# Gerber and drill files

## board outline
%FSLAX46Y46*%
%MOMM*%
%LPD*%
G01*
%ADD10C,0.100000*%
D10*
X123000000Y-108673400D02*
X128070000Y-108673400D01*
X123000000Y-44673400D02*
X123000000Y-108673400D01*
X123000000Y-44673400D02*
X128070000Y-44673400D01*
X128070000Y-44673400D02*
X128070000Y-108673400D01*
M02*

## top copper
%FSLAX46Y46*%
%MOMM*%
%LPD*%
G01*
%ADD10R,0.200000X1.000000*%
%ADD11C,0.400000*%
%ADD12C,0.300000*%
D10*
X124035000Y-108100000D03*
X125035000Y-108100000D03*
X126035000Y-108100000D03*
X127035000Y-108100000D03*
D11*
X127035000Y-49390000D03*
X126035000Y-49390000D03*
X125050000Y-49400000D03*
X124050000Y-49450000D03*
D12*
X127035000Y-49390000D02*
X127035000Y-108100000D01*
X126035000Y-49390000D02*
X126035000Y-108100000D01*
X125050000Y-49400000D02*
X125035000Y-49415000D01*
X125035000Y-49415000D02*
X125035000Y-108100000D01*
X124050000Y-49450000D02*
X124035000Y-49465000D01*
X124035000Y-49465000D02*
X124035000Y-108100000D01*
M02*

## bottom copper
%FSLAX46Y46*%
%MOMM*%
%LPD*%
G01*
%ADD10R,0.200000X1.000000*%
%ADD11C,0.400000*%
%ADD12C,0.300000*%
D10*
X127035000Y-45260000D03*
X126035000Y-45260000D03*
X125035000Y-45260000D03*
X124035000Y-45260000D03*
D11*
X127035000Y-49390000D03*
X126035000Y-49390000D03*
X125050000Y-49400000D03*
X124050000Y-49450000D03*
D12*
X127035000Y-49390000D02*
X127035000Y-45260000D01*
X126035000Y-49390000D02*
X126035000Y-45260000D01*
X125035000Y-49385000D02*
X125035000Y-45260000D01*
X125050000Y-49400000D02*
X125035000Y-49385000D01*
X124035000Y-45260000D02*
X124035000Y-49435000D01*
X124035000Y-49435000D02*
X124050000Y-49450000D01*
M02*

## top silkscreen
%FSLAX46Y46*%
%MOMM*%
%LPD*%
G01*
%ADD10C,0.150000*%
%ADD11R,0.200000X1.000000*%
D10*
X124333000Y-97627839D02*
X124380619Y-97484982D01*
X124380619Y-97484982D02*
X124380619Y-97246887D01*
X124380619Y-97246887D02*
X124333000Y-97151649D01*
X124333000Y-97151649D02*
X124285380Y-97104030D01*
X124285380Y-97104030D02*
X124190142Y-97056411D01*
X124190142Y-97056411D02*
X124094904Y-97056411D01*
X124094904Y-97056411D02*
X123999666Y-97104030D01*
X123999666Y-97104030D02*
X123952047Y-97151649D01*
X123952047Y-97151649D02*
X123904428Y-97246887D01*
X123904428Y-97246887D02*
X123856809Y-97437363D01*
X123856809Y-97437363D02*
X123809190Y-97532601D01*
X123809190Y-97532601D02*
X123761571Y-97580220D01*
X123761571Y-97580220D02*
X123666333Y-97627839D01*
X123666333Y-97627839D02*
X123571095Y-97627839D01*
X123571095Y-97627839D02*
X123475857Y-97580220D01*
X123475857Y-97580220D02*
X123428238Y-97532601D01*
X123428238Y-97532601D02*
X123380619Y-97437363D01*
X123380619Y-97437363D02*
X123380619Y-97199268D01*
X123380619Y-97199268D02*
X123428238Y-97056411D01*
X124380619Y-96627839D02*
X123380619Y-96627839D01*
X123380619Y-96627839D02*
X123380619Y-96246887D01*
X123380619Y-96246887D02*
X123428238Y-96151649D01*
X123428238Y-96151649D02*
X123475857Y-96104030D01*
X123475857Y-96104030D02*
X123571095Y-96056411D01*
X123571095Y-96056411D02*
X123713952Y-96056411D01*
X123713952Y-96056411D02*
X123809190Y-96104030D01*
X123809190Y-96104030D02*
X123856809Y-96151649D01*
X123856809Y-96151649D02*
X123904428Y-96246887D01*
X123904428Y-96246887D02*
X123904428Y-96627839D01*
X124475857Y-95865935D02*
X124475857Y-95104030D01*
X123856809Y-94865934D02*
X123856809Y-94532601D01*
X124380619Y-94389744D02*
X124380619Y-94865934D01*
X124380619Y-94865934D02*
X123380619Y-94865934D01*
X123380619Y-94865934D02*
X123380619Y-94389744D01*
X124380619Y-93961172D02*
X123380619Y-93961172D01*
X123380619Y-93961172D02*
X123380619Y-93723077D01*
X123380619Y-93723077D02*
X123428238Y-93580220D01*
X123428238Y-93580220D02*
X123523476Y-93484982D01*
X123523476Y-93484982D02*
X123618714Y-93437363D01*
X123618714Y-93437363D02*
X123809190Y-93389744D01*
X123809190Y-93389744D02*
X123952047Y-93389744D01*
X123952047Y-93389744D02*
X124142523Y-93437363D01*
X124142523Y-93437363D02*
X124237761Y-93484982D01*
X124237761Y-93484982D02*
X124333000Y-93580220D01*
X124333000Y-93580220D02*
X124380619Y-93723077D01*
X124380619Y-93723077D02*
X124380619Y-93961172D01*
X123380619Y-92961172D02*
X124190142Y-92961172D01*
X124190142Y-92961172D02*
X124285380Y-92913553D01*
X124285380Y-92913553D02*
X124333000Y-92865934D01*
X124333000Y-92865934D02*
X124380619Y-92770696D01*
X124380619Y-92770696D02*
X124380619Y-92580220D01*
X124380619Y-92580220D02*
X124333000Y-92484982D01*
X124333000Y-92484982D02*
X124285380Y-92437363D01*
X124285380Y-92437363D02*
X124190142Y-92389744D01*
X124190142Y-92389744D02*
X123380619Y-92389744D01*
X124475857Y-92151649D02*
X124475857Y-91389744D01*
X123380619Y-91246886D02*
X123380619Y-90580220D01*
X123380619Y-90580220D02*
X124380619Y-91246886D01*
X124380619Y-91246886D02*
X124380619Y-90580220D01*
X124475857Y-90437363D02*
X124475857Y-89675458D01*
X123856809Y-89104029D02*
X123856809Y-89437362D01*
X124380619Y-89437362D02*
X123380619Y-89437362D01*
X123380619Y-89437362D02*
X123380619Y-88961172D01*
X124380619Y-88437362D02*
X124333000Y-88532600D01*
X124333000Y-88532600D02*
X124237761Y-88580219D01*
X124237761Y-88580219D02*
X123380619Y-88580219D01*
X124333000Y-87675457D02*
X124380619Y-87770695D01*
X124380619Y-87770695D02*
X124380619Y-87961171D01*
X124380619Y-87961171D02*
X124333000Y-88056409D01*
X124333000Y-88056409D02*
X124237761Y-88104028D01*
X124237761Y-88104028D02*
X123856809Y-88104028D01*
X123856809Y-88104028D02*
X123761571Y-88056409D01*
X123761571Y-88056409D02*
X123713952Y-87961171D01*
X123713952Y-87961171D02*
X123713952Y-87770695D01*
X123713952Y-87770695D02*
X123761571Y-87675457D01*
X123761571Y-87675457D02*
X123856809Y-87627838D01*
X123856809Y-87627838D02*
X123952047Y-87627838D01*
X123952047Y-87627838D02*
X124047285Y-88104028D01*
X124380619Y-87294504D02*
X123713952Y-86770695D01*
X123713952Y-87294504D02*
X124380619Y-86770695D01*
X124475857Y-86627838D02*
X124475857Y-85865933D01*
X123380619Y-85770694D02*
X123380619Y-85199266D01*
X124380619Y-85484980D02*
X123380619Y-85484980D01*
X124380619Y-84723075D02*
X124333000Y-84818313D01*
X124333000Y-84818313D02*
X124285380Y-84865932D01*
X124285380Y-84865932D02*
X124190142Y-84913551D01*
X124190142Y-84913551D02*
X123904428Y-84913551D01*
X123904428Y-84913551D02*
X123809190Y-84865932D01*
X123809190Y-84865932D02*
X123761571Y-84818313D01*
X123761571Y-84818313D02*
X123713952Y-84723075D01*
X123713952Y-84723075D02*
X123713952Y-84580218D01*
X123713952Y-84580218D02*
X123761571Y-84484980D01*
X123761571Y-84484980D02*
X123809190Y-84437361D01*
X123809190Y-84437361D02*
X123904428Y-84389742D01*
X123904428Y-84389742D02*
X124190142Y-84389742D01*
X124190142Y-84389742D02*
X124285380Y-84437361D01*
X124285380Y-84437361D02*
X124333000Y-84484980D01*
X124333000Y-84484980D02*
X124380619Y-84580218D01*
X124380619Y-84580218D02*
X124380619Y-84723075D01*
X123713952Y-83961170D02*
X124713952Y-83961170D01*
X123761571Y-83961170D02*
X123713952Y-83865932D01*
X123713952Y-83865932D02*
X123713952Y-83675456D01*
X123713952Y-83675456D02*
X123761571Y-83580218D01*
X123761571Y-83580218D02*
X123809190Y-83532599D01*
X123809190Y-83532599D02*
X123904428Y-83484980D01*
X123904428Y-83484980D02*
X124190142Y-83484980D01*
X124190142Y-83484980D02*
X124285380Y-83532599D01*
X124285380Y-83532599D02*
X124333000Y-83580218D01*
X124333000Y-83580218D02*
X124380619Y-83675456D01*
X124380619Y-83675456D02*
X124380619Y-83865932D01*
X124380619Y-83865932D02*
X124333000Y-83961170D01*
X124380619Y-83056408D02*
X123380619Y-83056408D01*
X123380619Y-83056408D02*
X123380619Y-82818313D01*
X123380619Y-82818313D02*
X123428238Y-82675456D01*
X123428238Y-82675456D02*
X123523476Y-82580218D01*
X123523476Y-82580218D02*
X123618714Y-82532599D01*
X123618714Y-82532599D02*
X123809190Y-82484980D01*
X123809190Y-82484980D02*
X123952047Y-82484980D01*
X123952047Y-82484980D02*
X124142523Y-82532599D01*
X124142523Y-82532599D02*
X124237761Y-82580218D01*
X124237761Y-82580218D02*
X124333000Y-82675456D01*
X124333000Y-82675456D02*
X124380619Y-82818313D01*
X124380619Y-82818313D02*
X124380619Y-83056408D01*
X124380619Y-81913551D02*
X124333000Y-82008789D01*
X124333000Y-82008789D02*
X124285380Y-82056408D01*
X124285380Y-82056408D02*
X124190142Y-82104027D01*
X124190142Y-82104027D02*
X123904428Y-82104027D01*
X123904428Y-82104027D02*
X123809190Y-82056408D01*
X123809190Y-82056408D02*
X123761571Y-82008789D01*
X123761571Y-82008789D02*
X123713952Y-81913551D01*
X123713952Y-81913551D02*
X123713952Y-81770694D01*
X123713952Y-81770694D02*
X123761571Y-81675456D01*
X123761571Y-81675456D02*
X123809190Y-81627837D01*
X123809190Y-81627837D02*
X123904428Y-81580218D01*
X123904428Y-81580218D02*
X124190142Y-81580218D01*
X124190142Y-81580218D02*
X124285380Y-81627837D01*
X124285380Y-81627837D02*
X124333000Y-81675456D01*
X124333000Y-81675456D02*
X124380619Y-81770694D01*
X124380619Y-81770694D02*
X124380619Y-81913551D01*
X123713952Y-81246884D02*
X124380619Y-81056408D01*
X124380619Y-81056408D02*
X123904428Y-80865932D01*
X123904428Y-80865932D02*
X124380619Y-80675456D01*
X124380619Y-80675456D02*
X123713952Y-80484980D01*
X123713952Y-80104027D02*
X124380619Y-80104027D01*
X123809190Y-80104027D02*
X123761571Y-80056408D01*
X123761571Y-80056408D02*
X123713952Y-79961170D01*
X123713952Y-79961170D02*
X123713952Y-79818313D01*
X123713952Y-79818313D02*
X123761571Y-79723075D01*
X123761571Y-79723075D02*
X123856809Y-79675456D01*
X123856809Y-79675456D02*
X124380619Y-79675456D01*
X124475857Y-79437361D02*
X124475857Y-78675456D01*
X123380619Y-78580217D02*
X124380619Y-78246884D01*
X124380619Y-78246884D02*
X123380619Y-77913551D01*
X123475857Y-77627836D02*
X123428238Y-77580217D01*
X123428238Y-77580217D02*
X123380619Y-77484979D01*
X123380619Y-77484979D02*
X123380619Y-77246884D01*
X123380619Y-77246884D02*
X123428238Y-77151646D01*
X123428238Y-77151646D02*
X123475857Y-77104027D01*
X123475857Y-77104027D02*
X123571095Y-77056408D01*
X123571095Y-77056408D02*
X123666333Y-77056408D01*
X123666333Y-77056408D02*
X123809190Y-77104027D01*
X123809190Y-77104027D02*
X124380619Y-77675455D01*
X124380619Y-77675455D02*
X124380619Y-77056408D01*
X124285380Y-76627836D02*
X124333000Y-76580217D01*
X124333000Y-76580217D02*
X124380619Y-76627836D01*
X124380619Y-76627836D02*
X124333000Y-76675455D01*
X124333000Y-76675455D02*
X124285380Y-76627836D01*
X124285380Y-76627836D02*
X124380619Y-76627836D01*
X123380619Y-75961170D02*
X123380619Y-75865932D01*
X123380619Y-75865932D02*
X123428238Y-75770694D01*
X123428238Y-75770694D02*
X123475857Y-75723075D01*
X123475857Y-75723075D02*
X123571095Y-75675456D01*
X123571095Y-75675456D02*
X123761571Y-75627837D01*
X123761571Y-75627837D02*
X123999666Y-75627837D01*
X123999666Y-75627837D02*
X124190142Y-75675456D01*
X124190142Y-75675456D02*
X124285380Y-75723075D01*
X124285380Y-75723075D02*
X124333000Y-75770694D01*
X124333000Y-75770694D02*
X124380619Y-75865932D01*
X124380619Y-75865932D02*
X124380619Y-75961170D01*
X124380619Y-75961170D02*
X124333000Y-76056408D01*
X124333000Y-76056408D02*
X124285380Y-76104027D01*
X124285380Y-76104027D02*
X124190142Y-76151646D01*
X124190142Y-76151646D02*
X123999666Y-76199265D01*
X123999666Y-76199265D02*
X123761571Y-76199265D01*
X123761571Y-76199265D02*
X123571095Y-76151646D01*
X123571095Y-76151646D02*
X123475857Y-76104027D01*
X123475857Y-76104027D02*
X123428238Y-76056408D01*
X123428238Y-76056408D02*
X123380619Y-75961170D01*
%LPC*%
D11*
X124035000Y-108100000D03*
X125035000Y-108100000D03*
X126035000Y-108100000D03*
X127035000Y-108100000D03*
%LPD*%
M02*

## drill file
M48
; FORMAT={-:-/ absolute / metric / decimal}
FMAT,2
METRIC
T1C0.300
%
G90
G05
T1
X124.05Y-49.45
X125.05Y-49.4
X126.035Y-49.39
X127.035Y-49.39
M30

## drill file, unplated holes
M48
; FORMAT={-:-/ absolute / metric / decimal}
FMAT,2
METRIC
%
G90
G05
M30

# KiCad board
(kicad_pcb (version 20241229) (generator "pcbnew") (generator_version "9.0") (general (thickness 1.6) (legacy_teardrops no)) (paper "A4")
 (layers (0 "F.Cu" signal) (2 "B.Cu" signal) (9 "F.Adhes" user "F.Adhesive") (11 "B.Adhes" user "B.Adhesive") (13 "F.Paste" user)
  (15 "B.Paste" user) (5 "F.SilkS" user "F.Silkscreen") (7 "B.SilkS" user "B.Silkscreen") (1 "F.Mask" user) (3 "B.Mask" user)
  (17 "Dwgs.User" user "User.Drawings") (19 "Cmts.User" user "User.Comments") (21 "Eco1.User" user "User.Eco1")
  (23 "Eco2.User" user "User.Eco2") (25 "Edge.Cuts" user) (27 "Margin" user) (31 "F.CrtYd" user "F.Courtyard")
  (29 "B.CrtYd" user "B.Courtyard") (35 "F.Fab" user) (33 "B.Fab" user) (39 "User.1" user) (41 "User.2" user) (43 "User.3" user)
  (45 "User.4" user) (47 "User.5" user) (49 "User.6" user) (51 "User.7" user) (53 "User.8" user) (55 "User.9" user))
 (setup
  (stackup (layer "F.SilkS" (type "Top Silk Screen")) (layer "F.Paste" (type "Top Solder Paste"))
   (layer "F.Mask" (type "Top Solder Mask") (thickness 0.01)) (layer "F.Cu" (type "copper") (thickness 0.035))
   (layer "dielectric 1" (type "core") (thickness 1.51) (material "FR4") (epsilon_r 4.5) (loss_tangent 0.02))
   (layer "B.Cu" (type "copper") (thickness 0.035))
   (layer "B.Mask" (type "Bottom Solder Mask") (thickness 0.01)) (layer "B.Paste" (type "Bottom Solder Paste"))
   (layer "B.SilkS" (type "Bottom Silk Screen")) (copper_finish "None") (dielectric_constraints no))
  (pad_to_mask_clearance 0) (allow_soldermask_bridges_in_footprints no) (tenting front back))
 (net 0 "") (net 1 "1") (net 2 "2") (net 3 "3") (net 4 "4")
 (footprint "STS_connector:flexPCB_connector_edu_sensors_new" (layer "F.Cu") (at 123.535 107.6)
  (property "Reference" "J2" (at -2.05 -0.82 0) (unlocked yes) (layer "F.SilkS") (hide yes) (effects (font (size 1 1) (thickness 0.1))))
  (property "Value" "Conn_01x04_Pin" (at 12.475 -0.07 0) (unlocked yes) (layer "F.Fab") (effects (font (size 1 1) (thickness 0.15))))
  (pad "1" smd rect (at 0.5 0.5) (size 0.2 1) (layers "F.Cu" "F.Mask" "F.Paste") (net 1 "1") (thermal_bridge_angle 45))
  (pad "2" smd rect (at 1.5 0.5) (size 0.2 1) (layers "F.Cu" "F.Mask" "F.Paste") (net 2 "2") (thermal_bridge_angle 45))
  (pad "3" smd rect (at 2.5 0.5) (size 0.2 1) (layers "F.Cu" "F.Mask" "F.Paste") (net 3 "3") (thermal_bridge_angle 45))
  (pad "4" smd rect (at 3.5 0.5) (size 0.2 1) (layers "F.Cu" "F.Mask" "F.Paste") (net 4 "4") (thermal_bridge_angle 45)))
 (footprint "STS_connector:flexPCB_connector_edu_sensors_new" (layer "B.Cu") (at 127.535 44.76 180)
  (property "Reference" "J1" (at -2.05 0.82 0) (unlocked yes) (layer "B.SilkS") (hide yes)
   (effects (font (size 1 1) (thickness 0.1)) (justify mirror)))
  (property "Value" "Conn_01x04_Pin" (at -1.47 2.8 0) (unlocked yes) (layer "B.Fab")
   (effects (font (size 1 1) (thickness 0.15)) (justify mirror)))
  (pad "1" smd rect (at 0.5 -0.5 180) (size 0.2 1) (layers "B.Cu" "B.Mask" "B.Paste") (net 4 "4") (thermal_bridge_angle 45))
  (pad "2" smd rect (at 1.5 -0.5 180) (size 0.2 1) (layers "B.Cu" "B.Mask" "B.Paste") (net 3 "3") (thermal_bridge_angle 45))
  (pad "3" smd rect (at 2.5 -0.5 180) (size 0.2 1) (layers "B.Cu" "B.Mask" "B.Paste") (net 2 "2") (thermal_bridge_angle 45))
  (pad "4" smd rect (at 3.5 -0.5 180) (size 0.2 1) (layers "B.Cu" "B.Mask" "B.Paste") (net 1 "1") (thermal_bridge_angle 45)))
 (gr_line (start 123 108.6734) (end 128.07 108.6734) (stroke (width 0.1) (type solid)) (layer "Edge.Cuts"))
 (gr_line (start 123 44.6734) (end 123 108.6734) (stroke (width 0.1) (type solid)) (layer "Edge.Cuts"))
 (gr_line (start 123 44.6734) (end 128.07 44.6734) (stroke (width 0.1) (type solid)) (layer "Edge.Cuts"))
 (gr_line (start 128.07 44.6734) (end 128.07 108.6734) (stroke (width 0.1) (type solid)) (layer "Edge.Cuts"))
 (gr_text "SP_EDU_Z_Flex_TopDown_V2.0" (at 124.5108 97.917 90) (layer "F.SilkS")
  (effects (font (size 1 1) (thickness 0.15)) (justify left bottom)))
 (segment (start 127.035 49.39) (end 127.035 108.1) (width 0.3) (layer "F.Cu") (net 4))
 (via (at 127.035 49.39) (size 0.4) (drill 0.3) (layers "F.Cu" "B.Cu") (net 4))
 (segment (start 127.035 49.39) (end 127.035 45.26) (width 0.3) (layer "B.Cu") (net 4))
 (segment (start 126.035 49.39) (end 126.035 108.1) (width 0.3) (layer "F.Cu") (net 3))
 (via (at 126.035 49.39) (size 0.4) (drill 0.3) (layers "F.Cu" "B.Cu") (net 3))
 (segment (start 126.035 49.39) (end 126.035 45.26) (width 0.3) (layer "B.Cu") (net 3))
 (segment (start 125.05 49.4) (end 125.035 49.415) (width 0.3) (layer "F.Cu") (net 2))
 (segment (start 125.035 49.415) (end 125.035 108.1) (width 0.3) (layer "F.Cu") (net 2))
 (via (at 125.05 49.4) (size 0.4) (drill 0.3) (layers "F.Cu" "B.Cu") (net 2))
 (segment (start 125.035 49.385) (end 125.035 45.26) (width 0.3) (layer "B.Cu") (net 2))
 (segment (start 125.05 49.4) (end 125.035 49.385) (width 0.3) (layer "B.Cu") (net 2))
 (segment (start 124.05 49.45) (end 124.035 49.465) (width 0.3) (layer "F.Cu") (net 1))
 (segment (start 124.035 49.465) (end 124.035 108.1) (width 0.3) (layer "F.Cu") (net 1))
 (via (at 124.05 49.45) (size 0.4) (drill 0.3) (layers "F.Cu" "B.Cu") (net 1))
 (segment (start 124.035 45.26) (end 124.035 49.435) (width 0.3) (layer "B.Cu") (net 1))
 (segment (start 124.035 49.435) (end 124.05 49.45) (width 0.3) (layer "B.Cu") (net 1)))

